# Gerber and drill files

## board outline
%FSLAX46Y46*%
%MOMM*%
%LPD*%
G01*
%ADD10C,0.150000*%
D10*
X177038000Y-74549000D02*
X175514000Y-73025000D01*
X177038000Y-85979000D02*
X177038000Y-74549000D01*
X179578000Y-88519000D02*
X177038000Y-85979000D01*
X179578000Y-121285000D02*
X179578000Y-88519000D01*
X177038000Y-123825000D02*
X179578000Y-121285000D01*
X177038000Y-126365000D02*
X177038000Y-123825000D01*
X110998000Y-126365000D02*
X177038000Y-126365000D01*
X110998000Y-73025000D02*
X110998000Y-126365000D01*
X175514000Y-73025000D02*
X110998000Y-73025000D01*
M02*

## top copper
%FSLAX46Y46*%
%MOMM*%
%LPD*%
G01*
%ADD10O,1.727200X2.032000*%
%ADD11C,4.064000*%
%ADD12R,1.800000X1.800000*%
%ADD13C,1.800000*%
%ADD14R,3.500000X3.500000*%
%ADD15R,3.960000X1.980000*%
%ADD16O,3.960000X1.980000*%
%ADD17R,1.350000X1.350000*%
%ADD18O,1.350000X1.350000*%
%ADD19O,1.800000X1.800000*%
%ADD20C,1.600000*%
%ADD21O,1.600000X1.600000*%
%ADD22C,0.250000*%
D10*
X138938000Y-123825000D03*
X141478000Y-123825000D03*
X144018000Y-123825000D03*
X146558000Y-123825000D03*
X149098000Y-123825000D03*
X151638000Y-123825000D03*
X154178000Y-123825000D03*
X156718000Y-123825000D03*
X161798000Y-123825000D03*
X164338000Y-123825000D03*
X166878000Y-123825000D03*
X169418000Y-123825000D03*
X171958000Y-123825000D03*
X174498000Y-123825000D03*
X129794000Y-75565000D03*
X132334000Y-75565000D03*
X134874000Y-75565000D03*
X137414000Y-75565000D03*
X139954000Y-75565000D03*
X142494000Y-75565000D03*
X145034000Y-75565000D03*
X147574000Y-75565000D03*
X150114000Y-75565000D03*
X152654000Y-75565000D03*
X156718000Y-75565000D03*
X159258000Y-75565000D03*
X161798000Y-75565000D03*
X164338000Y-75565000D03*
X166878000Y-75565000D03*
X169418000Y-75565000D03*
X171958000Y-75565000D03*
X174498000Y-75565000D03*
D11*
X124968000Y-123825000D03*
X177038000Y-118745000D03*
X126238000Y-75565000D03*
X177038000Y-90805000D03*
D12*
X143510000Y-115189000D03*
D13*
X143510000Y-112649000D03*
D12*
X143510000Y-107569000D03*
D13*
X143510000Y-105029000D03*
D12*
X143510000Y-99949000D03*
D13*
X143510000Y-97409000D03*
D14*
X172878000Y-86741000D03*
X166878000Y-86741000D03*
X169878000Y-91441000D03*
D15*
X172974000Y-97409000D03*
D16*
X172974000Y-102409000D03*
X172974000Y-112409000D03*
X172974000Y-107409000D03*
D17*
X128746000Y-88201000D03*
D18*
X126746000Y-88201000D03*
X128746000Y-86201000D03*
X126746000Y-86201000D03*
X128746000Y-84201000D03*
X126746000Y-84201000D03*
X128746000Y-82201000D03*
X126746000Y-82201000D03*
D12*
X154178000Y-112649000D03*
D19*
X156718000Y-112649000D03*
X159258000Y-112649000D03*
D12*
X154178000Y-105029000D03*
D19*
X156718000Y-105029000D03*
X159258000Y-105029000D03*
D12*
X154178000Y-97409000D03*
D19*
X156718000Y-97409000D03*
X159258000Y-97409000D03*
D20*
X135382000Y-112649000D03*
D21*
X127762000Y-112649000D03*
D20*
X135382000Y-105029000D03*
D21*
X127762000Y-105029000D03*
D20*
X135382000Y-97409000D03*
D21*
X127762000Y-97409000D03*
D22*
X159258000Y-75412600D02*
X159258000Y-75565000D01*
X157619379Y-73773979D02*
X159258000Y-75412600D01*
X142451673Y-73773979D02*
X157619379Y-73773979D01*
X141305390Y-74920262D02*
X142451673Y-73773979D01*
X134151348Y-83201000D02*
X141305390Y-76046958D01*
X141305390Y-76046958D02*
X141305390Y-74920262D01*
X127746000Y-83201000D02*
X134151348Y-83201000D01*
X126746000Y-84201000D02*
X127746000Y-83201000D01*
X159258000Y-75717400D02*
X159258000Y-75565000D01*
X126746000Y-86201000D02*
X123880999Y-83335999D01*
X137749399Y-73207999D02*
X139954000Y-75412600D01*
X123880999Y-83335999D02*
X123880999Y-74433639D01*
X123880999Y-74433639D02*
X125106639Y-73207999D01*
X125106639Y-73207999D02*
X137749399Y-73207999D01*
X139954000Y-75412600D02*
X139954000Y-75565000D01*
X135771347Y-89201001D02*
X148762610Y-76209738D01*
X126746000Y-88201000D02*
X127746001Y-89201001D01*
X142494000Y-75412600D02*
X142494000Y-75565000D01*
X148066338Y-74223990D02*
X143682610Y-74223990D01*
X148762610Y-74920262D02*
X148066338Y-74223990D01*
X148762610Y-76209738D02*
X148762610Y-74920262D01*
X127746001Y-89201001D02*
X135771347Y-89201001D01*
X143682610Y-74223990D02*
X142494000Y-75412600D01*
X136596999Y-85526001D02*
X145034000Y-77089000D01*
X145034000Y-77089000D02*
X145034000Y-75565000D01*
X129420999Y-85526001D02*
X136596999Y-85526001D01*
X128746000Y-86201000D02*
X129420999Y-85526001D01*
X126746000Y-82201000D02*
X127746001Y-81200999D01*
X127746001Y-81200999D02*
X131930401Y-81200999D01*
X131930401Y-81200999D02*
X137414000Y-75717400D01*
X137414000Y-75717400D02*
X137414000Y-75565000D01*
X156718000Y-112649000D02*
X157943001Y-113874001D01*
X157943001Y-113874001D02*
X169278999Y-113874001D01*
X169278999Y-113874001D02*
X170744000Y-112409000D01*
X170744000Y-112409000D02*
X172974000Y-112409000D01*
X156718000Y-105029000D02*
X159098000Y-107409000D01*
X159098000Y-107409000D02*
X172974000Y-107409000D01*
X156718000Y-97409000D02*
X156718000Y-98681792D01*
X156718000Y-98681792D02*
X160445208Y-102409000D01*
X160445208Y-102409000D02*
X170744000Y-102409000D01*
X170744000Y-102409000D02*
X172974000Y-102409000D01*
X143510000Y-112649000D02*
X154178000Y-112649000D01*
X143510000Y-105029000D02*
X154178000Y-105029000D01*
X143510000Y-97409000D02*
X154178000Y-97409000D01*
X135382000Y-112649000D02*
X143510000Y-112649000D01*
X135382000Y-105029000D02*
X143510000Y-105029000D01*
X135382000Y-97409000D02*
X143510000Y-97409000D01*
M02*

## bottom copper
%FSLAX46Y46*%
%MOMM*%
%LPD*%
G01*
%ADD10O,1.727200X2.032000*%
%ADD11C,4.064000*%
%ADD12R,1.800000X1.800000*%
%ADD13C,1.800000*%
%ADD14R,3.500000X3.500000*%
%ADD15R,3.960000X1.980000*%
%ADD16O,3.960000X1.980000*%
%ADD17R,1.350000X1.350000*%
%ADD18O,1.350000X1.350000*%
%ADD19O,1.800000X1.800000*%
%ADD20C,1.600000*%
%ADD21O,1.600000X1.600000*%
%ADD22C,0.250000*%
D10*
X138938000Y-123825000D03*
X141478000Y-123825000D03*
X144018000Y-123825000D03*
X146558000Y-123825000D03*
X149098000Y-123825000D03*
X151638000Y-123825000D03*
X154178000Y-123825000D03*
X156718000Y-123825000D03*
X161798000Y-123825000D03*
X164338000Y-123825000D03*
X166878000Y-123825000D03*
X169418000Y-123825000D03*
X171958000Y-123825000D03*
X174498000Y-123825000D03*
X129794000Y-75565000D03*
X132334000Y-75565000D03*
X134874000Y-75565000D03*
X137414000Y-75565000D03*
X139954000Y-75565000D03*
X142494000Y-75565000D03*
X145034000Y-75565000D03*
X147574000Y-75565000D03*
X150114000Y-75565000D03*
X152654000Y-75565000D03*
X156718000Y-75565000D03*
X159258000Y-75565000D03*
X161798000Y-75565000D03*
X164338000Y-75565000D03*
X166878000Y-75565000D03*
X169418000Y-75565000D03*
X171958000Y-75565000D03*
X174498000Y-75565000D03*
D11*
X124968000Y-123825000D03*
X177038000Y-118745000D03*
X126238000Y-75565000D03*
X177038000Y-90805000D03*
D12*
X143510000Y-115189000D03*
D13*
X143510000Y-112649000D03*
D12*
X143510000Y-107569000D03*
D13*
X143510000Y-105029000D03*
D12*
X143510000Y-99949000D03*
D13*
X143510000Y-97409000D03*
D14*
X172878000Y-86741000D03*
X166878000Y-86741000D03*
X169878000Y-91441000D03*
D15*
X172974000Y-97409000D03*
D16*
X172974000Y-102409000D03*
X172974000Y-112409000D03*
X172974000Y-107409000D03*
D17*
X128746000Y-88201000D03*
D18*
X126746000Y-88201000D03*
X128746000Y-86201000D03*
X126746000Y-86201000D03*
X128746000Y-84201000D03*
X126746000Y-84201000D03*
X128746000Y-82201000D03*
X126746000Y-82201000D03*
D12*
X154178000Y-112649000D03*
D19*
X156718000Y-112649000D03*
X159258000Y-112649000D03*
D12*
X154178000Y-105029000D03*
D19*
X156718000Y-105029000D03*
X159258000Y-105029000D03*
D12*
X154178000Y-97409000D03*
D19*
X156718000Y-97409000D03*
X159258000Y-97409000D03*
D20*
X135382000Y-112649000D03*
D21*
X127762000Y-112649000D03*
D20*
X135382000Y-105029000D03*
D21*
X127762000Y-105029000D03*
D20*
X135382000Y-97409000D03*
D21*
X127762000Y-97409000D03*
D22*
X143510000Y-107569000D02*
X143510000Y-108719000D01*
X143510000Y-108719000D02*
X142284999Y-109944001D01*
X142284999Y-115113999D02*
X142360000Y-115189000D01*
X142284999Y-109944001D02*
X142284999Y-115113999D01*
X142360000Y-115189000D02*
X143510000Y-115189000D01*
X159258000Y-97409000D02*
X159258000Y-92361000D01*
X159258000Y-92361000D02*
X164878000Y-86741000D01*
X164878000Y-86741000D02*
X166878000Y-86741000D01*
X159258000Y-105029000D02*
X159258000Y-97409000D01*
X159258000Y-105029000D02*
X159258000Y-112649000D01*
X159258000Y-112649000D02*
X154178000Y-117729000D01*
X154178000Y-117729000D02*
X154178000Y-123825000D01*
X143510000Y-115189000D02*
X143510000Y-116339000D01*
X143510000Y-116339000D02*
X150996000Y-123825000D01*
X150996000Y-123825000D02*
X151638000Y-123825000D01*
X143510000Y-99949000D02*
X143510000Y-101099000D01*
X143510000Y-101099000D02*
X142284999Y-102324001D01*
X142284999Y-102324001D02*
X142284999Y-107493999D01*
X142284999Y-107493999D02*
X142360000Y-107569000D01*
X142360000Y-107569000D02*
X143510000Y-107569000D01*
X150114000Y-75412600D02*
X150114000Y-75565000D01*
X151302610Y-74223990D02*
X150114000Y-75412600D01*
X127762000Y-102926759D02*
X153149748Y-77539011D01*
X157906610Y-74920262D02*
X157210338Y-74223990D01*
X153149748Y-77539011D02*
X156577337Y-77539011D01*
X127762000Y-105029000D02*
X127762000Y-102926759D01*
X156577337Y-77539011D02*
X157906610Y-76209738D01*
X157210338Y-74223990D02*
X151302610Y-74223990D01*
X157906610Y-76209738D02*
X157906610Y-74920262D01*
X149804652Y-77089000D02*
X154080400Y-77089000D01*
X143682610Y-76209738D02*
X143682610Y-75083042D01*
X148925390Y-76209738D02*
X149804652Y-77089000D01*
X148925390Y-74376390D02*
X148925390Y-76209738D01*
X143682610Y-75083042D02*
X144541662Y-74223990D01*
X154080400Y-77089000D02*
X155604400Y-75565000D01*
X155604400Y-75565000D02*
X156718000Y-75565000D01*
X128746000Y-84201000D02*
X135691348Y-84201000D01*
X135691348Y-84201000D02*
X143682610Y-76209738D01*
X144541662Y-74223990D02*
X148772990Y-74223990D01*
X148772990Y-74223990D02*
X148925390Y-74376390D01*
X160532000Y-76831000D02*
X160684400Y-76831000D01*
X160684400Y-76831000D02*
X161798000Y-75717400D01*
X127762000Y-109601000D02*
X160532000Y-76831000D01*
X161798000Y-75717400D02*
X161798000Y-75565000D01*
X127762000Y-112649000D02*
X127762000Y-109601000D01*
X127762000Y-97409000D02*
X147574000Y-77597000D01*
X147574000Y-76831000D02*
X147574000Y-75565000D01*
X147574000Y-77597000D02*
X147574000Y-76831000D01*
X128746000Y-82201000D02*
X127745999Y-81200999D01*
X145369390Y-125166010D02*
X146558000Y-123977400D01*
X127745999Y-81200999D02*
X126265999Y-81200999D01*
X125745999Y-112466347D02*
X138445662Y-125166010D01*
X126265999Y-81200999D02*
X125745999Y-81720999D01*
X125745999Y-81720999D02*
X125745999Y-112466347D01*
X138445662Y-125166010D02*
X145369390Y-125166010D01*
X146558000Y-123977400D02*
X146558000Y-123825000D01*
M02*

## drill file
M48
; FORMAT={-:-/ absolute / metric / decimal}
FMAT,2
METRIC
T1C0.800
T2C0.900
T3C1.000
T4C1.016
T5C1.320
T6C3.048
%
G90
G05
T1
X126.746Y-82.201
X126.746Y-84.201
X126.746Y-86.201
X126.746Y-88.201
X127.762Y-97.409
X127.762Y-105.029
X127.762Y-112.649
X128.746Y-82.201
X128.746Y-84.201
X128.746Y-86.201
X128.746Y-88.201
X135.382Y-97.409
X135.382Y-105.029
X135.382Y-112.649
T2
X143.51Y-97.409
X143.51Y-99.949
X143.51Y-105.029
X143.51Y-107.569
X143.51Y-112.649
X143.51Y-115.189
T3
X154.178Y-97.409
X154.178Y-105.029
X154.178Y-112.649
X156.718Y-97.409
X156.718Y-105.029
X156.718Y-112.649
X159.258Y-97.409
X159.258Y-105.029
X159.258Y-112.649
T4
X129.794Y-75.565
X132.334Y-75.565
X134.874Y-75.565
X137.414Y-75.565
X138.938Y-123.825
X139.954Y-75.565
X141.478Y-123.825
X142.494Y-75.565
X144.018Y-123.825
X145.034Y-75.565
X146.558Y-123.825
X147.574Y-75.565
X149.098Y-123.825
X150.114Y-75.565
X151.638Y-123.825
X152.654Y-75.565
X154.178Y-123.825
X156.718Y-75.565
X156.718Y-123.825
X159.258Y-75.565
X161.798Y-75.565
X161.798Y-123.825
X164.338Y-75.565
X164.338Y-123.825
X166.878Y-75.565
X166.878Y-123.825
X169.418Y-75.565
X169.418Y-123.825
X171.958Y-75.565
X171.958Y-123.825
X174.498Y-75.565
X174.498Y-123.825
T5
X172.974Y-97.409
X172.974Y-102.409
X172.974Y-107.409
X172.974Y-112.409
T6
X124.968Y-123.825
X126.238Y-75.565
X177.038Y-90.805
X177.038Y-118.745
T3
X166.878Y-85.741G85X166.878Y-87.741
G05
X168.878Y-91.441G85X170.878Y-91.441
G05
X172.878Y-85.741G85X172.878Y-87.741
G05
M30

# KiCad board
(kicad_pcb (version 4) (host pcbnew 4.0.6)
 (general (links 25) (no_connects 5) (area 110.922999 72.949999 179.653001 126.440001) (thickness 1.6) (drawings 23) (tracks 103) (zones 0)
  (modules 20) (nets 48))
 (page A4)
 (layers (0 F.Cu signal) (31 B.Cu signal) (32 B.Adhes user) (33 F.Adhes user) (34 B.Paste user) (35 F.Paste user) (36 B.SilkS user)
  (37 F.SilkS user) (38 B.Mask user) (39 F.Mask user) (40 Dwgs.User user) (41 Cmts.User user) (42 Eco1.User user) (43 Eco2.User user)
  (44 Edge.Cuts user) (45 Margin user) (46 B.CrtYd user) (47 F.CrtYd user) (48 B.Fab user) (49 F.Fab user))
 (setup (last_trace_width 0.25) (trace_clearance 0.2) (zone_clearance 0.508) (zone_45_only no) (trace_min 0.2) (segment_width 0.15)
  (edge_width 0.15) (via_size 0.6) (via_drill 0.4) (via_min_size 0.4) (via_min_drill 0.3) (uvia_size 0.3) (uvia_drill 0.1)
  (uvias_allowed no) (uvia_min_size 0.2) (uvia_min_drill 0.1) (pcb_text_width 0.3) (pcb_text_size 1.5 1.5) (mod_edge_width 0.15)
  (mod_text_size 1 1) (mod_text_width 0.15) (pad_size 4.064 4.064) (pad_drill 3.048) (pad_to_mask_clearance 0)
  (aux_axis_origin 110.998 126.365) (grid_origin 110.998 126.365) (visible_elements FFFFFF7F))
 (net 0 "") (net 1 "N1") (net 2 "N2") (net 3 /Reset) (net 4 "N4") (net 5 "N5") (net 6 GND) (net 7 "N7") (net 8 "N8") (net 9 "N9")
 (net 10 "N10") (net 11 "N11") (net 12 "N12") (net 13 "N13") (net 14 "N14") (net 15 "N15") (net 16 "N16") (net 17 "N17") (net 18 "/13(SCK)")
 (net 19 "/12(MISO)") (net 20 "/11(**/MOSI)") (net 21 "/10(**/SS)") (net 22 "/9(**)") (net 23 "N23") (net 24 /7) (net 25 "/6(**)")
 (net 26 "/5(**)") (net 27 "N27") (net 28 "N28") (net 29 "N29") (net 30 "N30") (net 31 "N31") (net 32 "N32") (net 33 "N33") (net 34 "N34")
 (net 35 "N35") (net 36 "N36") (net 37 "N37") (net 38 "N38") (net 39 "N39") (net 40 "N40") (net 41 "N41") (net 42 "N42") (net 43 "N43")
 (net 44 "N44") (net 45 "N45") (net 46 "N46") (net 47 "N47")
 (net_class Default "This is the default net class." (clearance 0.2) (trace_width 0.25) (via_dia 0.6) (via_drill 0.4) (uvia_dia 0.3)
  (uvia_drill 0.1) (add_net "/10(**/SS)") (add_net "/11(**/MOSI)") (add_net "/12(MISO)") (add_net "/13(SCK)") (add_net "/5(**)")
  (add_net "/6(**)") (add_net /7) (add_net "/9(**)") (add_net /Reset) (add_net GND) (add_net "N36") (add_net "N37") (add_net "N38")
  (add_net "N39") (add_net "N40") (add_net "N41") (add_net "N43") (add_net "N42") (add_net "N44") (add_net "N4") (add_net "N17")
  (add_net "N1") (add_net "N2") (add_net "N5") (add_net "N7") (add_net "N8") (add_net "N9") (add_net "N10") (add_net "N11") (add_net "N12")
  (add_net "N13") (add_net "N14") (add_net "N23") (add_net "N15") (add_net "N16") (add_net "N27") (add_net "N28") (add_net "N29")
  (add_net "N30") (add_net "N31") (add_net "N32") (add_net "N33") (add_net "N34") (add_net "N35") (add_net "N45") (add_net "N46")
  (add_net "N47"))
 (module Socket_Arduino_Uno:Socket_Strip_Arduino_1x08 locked (layer F.Cu) (at 138.938 123.825)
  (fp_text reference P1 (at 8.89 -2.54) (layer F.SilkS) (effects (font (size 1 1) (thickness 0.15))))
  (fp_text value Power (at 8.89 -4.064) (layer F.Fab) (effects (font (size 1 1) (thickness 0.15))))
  (pad 1 thru_hole oval (at 0 0) (size 1.7272 2.032) (drill 1.016) (layers *.Cu *.Mask F.SilkS) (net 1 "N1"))
  (pad 2 thru_hole oval (at 2.54 0) (size 1.7272 2.032) (drill 1.016) (layers *.Cu *.Mask F.SilkS) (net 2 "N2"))
  (pad 3 thru_hole oval (at 5.08 0) (size 1.7272 2.032) (drill 1.016) (layers *.Cu *.Mask F.SilkS) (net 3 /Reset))
  (pad 4 thru_hole oval (at 7.62 0) (size 1.7272 2.032) (drill 1.016) (layers *.Cu *.Mask F.SilkS) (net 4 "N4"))
  (pad 5 thru_hole oval (at 10.16 0) (size 1.7272 2.032) (drill 1.016) (layers *.Cu *.Mask F.SilkS) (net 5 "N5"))
  (pad 6 thru_hole oval (at 12.7 0) (size 1.7272 2.032) (drill 1.016) (layers *.Cu *.Mask F.SilkS) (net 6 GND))
  (pad 7 thru_hole oval (at 15.24 0) (size 1.7272 2.032) (drill 1.016) (layers *.Cu *.Mask F.SilkS) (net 6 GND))
  (pad 8 thru_hole oval (at 17.78 0) (size 1.7272 2.032) (drill 1.016) (layers *.Cu *.Mask F.SilkS) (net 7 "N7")))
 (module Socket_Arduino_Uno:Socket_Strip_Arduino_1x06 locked (layer F.Cu) (at 161.798 123.825)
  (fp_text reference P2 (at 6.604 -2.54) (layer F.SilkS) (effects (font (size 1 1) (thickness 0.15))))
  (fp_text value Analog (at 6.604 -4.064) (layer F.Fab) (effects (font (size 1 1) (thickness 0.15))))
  (pad 1 thru_hole oval (at 0 0) (size 1.7272 2.032) (drill 1.016) (layers *.Cu *.Mask F.SilkS) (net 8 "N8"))
  (pad 2 thru_hole oval (at 2.54 0) (size 1.7272 2.032) (drill 1.016) (layers *.Cu *.Mask F.SilkS) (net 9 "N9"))
  (pad 3 thru_hole oval (at 5.08 0) (size 1.7272 2.032) (drill 1.016) (layers *.Cu *.Mask F.SilkS) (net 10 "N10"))
  (pad 4 thru_hole oval (at 7.62 0) (size 1.7272 2.032) (drill 1.016) (layers *.Cu *.Mask F.SilkS) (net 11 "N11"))
  (pad 5 thru_hole oval (at 10.16 0) (size 1.7272 2.032) (drill 1.016) (layers *.Cu *.Mask F.SilkS) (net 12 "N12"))
  (pad 6 thru_hole oval (at 12.7 0) (size 1.7272 2.032) (drill 1.016) (layers *.Cu *.Mask F.SilkS) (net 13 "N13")))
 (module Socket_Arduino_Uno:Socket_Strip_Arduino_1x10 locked (layer F.Cu) (at 129.794 75.565)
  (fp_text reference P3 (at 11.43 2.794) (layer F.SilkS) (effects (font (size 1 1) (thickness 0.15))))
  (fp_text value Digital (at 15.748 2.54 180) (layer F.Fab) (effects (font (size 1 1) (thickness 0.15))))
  (pad 1 thru_hole oval (at 0 0) (size 1.7272 2.032) (drill 1.016) (layers *.Cu *.Mask F.SilkS) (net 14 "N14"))
  (pad 2 thru_hole oval (at 2.54 0) (size 1.7272 2.032) (drill 1.016) (layers *.Cu *.Mask F.SilkS) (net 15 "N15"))
  (pad 3 thru_hole oval (at 5.08 0) (size 1.7272 2.032) (drill 1.016) (layers *.Cu *.Mask F.SilkS) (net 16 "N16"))
  (pad 4 thru_hole oval (at 7.62 0) (size 1.7272 2.032) (drill 1.016) (layers *.Cu *.Mask F.SilkS) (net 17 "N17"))
  (pad 5 thru_hole oval (at 10.16 0) (size 1.7272 2.032) (drill 1.016) (layers *.Cu *.Mask F.SilkS) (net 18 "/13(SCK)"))
  (pad 6 thru_hole oval (at 12.7 0) (size 1.7272 2.032) (drill 1.016) (layers *.Cu *.Mask F.SilkS) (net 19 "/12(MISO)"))
  (pad 7 thru_hole oval (at 15.24 0) (size 1.7272 2.032) (drill 1.016) (layers *.Cu *.Mask F.SilkS) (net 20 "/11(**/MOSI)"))
  (pad 8 thru_hole oval (at 17.78 0) (size 1.7272 2.032) (drill 1.016) (layers *.Cu *.Mask F.SilkS) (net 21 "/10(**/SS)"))
  (pad 9 thru_hole oval (at 20.32 0) (size 1.7272 2.032) (drill 1.016) (layers *.Cu *.Mask F.SilkS) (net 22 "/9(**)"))
  (pad 10 thru_hole oval (at 22.86 0) (size 1.7272 2.032) (drill 1.016) (layers *.Cu *.Mask F.SilkS) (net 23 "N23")))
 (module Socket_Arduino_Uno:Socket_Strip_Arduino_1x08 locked (layer F.Cu) (at 156.718 75.565)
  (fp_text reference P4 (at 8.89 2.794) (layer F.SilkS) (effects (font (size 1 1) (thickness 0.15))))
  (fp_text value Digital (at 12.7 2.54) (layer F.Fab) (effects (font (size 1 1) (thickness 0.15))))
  (pad 1 thru_hole oval (at 0 0) (size 1.7272 2.032) (drill 1.016) (layers *.Cu *.Mask F.SilkS) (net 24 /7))
  (pad 2 thru_hole oval (at 2.54 0) (size 1.7272 2.032) (drill 1.016) (layers *.Cu *.Mask F.SilkS) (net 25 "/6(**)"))
  (pad 3 thru_hole oval (at 5.08 0) (size 1.7272 2.032) (drill 1.016) (layers *.Cu *.Mask F.SilkS) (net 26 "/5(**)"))
  (pad 4 thru_hole oval (at 7.62 0) (size 1.7272 2.032) (drill 1.016) (layers *.Cu *.Mask F.SilkS) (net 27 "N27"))
  (pad 5 thru_hole oval (at 10.16 0) (size 1.7272 2.032) (drill 1.016) (layers *.Cu *.Mask F.SilkS) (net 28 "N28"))
  (pad 6 thru_hole oval (at 12.7 0) (size 1.7272 2.032) (drill 1.016) (layers *.Cu *.Mask F.SilkS) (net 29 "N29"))
  (pad 7 thru_hole oval (at 15.24 0) (size 1.7272 2.032) (drill 1.016) (layers *.Cu *.Mask F.SilkS) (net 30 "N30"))
  (pad 8 thru_hole oval (at 17.78 0) (size 1.7272 2.032) (drill 1.016) (layers *.Cu *.Mask F.SilkS) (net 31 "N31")))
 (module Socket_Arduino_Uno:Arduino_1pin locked (layer F.Cu) (at 124.968 123.825)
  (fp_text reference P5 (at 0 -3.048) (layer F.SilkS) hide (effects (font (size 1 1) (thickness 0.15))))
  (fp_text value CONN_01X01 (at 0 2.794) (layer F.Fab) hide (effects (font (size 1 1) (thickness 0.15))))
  (pad 1 thru_hole circle (at 0 0) (size 4.064 4.064) (drill 3.048) (layers *.Cu *.Mask F.SilkS) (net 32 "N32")))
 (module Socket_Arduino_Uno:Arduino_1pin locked (layer F.Cu) (at 177.038 118.745)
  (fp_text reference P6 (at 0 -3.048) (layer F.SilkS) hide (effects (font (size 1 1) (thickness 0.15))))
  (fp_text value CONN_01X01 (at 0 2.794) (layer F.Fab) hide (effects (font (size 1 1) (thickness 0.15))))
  (pad 1 thru_hole circle (at 0 0) (size 4.064 4.064) (drill 3.048) (layers *.Cu *.Mask F.SilkS) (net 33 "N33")))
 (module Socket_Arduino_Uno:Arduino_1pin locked (layer F.Cu) (at 126.238 75.565)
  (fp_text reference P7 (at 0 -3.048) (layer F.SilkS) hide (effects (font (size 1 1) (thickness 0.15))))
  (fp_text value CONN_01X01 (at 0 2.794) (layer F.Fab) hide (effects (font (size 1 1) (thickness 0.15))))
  (pad 1 thru_hole circle (at 0 0) (size 4.064 4.064) (drill 3.048) (layers *.Cu *.Mask F.SilkS) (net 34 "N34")))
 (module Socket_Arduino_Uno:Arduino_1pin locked (layer F.Cu) (at 177.038 90.805)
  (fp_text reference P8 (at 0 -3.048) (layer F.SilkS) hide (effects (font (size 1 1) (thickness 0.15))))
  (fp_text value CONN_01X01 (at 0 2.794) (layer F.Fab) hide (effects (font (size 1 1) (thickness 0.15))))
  (pad 1 thru_hole circle (at 0 0) (size 4.064 4.064) (drill 3.048) (layers *.Cu *.Mask F.SilkS) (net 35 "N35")))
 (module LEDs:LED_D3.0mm (layer F.Cu) (at 143.51 115.189 90)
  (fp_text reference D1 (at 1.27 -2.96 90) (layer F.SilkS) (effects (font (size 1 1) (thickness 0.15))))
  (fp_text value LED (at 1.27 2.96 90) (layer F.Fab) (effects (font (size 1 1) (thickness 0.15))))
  (pad 1 thru_hole rect (at 0 0 90) (size 1.8 1.8) (drill 0.9) (layers *.Cu *.Mask) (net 6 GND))
  (pad 2 thru_hole circle (at 2.54 0 90) (size 1.8 1.8) (drill 0.9) (layers *.Cu *.Mask) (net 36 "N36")))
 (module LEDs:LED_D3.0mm (layer F.Cu) (at 143.51 107.569 90)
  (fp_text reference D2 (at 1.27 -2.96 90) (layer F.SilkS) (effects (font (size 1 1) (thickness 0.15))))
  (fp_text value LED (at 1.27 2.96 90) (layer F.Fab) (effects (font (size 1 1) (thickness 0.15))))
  (pad 1 thru_hole rect (at 0 0 90) (size 1.8 1.8) (drill 0.9) (layers *.Cu *.Mask) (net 6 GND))
  (pad 2 thru_hole circle (at 2.54 0 90) (size 1.8 1.8) (drill 0.9) (layers *.Cu *.Mask) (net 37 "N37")))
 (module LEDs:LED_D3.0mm (layer F.Cu) (at 143.51 99.949 90)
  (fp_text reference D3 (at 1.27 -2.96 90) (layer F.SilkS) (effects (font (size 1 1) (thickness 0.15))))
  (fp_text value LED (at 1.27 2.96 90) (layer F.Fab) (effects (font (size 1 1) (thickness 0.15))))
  (pad 1 thru_hole rect (at 0 0 90) (size 1.8 1.8) (drill 0.9) (layers *.Cu *.Mask) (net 6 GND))
  (pad 2 thru_hole circle (at 2.54 0 90) (size 1.8 1.8) (drill 0.9) (layers *.Cu *.Mask) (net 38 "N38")))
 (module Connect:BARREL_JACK (layer F.Cu) (at 172.878 86.741)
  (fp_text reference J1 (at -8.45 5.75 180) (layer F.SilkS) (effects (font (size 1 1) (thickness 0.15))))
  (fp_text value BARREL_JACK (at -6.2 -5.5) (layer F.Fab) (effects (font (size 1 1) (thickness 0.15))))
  (pad 1 thru_hole rect (at 0 0) (size 3.5 3.5) (drill oval 1 3) (layers *.Cu *.Mask) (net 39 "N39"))
  (pad 2 thru_hole rect (at -6 0) (size 3.5 3.5) (drill oval 1 3) (layers *.Cu *.Mask) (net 6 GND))
  (pad 3 thru_hole rect (at -3 4.7) (size 3.5 3.5) (drill oval 3 1) (layers *.Cu *.Mask) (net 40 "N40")))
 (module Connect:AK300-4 (layer F.Cu) (at 172.974 97.409 270)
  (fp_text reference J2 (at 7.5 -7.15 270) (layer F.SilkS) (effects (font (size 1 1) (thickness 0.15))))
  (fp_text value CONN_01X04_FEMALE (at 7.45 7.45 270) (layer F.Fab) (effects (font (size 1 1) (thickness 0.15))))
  (pad 1 thru_hole rect (at 0 0 270) (size 1.98 3.96) (drill 1.32) (layers *.Cu F.Paste F.Mask) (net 39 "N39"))
  (pad 2 thru_hole oval (at 5 0 270) (size 1.98 3.96) (drill 1.32) (layers *.Cu F.Paste F.Mask) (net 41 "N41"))
  (pad 4 thru_hole oval (at 15 0 270) (size 1.98 3.96) (drill 1.32) (layers *.Cu F.Paste F.Mask) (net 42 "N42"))
  (pad 3 thru_hole oval (at 10 0 270) (size 1.98 3.96) (drill 1.32) (layers *.Cu *.Mask) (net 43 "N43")))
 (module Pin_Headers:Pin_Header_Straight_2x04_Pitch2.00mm (layer F.Cu) (at 128.746 88.201 180)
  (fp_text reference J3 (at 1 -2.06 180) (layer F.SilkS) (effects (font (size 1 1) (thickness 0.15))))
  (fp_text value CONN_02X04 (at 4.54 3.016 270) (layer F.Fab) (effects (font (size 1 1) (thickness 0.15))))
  (pad 1 thru_hole rect (at 0 0 180) (size 1.35 1.35) (drill 0.8) (layers *.Cu *.Mask) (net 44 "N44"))
  (pad 2 thru_hole oval (at 2 0 180) (size 1.35 1.35) (drill 0.8) (layers *.Cu *.Mask) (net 19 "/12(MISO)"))
  (pad 3 thru_hole oval (at 0 2 180) (size 1.35 1.35) (drill 0.8) (layers *.Cu *.Mask) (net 20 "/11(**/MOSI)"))
  (pad 4 thru_hole oval (at 2 2 180) (size 1.35 1.35) (drill 0.8) (layers *.Cu *.Mask) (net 18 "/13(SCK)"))
  (pad 5 thru_hole oval (at 0 4 180) (size 1.35 1.35) (drill 0.8) (layers *.Cu *.Mask) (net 24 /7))
  (pad 6 thru_hole oval (at 2 4 180) (size 1.35 1.35) (drill 0.8) (layers *.Cu *.Mask) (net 25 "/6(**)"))
  (pad 7 thru_hole oval (at 0 6 180) (size 1.35 1.35) (drill 0.8) (layers *.Cu *.Mask) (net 4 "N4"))
  (pad 8 thru_hole oval (at 2 6 180) (size 1.35 1.35) (drill 0.8) (layers *.Cu *.Mask) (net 17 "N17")))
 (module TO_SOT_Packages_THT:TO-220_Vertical (layer F.Cu) (at 154.178 112.649)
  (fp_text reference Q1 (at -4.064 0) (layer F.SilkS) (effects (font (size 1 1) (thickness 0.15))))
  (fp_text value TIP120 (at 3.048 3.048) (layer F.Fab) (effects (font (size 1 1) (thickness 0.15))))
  (pad 1 thru_hole rect (at 0 0) (size 1.8 1.8) (drill 1) (layers *.Cu *.Mask) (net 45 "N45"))
  (pad 2 thru_hole oval (at 2.54 0) (size 1.8 1.8) (drill 1) (layers *.Cu *.Mask) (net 42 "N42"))
  (pad 3 thru_hole oval (at 5.08 0) (size 1.8 1.8) (drill 1) (layers *.Cu *.Mask) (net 6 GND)))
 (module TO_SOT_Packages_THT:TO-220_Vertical (layer F.Cu) (at 154.178 105.029)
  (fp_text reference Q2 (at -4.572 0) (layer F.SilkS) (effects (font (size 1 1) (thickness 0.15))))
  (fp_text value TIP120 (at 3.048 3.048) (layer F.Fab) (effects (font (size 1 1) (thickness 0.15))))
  (pad 1 thru_hole rect (at 0 0) (size 1.8 1.8) (drill 1) (layers *.Cu *.Mask) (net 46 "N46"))
  (pad 2 thru_hole oval (at 2.54 0) (size 1.8 1.8) (drill 1) (layers *.Cu *.Mask) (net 43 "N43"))
  (pad 3 thru_hole oval (at 5.08 0) (size 1.8 1.8) (drill 1) (layers *.Cu *.Mask) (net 6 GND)))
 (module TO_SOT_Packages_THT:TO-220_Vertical (layer F.Cu) (at 154.178 97.409)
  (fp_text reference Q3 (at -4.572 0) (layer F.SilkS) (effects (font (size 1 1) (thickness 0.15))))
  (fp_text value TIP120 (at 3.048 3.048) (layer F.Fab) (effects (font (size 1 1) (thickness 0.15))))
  (pad 1 thru_hole rect (at 0 0) (size 1.8 1.8) (drill 1) (layers *.Cu *.Mask) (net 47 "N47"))
  (pad 2 thru_hole oval (at 2.54 0) (size 1.8 1.8) (drill 1) (layers *.Cu *.Mask) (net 41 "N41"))
  (pad 3 thru_hole oval (at 5.08 0) (size 1.8 1.8) (drill 1) (layers *.Cu *.Mask) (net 6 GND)))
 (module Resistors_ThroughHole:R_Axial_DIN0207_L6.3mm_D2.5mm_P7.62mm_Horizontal (layer F.Cu) (at 135.382 112.649 180)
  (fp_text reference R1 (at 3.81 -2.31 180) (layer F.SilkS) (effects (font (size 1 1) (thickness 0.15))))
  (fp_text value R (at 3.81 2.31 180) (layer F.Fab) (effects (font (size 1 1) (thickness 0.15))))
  (pad 1 thru_hole circle (at 0 0 180) (size 1.6 1.6) (drill 0.8) (layers *.Cu *.Mask) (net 45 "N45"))
  (pad 2 thru_hole oval (at 7.62 0 180) (size 1.6 1.6) (drill 0.8) (layers *.Cu *.Mask) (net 26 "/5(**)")))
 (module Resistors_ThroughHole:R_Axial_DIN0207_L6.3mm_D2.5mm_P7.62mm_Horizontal (layer F.Cu) (at 135.382 105.029 180)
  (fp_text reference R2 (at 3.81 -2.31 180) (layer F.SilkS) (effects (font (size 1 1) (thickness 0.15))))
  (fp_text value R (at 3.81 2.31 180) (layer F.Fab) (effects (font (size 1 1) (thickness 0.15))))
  (pad 1 thru_hole circle (at 0 0 180) (size 1.6 1.6) (drill 0.8) (layers *.Cu *.Mask) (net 46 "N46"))
  (pad 2 thru_hole oval (at 7.62 0 180) (size 1.6 1.6) (drill 0.8) (layers *.Cu *.Mask) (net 22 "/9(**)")))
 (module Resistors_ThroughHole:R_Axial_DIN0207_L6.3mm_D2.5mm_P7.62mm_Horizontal (layer F.Cu) (at 135.382 97.409 180)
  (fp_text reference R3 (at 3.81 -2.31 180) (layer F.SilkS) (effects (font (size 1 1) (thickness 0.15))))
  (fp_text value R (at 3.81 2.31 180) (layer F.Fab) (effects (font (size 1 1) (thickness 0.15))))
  (pad 1 thru_hole circle (at 0 0 180) (size 1.6 1.6) (drill 0.8) (layers *.Cu *.Mask) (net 47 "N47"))
  (pad 2 thru_hole oval (at 7.62 0 180) (size 1.6 1.6) (drill 0.8) (layers *.Cu *.Mask) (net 21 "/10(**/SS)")))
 (gr_line (start 177.038 74.549) (end 175.514 73.025) (angle 90) (layer Edge.Cuts) (width 0.15))
 (gr_line (start 177.038 85.979) (end 177.038 74.549) (angle 90) (layer Edge.Cuts) (width 0.15))
 (gr_line (start 179.578 88.519) (end 177.038 85.979) (angle 90) (layer Edge.Cuts) (width 0.15))
 (gr_line (start 179.578 121.285) (end 179.578 88.519) (angle 90) (layer Edge.Cuts) (width 0.15))
 (gr_line (start 177.038 123.825) (end 179.578 121.285) (angle 90) (layer Edge.Cuts) (width 0.15))
 (gr_line (start 177.038 126.365) (end 177.038 123.825) (angle 90) (layer Edge.Cuts) (width 0.15))
 (gr_line (start 110.998 126.365) (end 177.038 126.365) (angle 90) (layer Edge.Cuts) (width 0.15))
 (gr_line (start 110.998 73.025) (end 110.998 126.365) (angle 90) (layer Edge.Cuts) (width 0.15))
 (gr_line (start 175.514 73.025) (end 110.998 73.025) (angle 90) (layer Edge.Cuts) (width 0.15))
 (segment (start 143.51 107.569) (end 143.51 108.719) (width 0.25) (layer B.Cu) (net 6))
 (segment (start 143.51 108.719) (end 142.284999 109.944001) (width 0.25) (layer B.Cu) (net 6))
 (segment (start 142.284999 115.113999) (end 142.36 115.189) (width 0.25) (layer B.Cu) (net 6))
 (segment (start 142.284999 109.944001) (end 142.284999 115.113999) (width 0.25) (layer B.Cu) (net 6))
 (segment (start 142.36 115.189) (end 143.51 115.189) (width 0.25) (layer B.Cu) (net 6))
 (segment (start 159.258 97.409) (end 159.258 92.361) (width 0.25) (layer B.Cu) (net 6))
 (segment (start 159.258 92.361) (end 164.878 86.741) (width 0.25) (layer B.Cu) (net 6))
 (segment (start 164.878 86.741) (end 166.878 86.741) (width 0.25) (layer B.Cu) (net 6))
 (segment (start 159.258 105.029) (end 159.258 97.409) (width 0.25) (layer B.Cu) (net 6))
 (segment (start 159.258 105.029) (end 159.258 112.649) (width 0.25) (layer B.Cu) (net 6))
 (segment (start 159.258 112.649) (end 154.178 117.729) (width 0.25) (layer B.Cu) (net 6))
 (segment (start 154.178 117.729) (end 154.178 123.825) (width 0.25) (layer B.Cu) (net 6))
 (segment (start 143.51 115.189) (end 143.51 116.339) (width 0.25) (layer B.Cu) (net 6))
 (segment (start 143.51 116.339) (end 150.996 123.825) (width 0.25) (layer B.Cu) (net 6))
 (segment (start 150.996 123.825) (end 151.638 123.825) (width 0.25) (layer B.Cu) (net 6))
 (segment (start 143.51 99.949) (end 143.51 101.099) (width 0.25) (layer B.Cu) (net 6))
 (segment (start 143.51 101.099) (end 142.284999 102.324001) (width 0.25) (layer B.Cu) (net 6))
 (segment (start 142.284999 102.324001) (end 142.284999 107.493999) (width 0.25) (layer B.Cu) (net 6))
 (segment (start 142.284999 107.493999) (end 142.36 107.569) (width 0.25) (layer B.Cu) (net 6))
 (segment (start 142.36 107.569) (end 143.51 107.569) (width 0.25) (layer B.Cu) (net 6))
 (segment (start 150.114 75.4126) (end 150.114 75.565) (width 0.25) (layer B.Cu) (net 22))
 (segment (start 151.30261 74.22399) (end 150.114 75.4126) (width 0.25) (layer B.Cu) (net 22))
 (segment (start 127.762 102.926759) (end 153.149748 77.539011) (width 0.25) (layer B.Cu) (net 22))
 (segment (start 157.90661 74.920262) (end 157.210338 74.22399) (width 0.25) (layer B.Cu) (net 22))
 (segment (start 153.149748 77.539011) (end 156.577337 77.539011) (width 0.25) (layer B.Cu) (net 22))
 (segment (start 127.762 105.029) (end 127.762 102.926759) (width 0.25) (layer B.Cu) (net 22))
 (segment (start 156.577337 77.539011) (end 157.90661 76.209738) (width 0.25) (layer B.Cu) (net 22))
 (segment (start 157.210338 74.22399) (end 151.30261 74.22399) (width 0.25) (layer B.Cu) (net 22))
 (segment (start 157.90661 76.209738) (end 157.90661 74.920262) (width 0.25) (layer B.Cu) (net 22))
 (segment (start 149.804652 77.089) (end 154.0804 77.089) (width 0.25) (layer B.Cu) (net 24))
 (segment (start 143.68261 76.209738) (end 143.68261 75.083042) (width 0.25) (layer B.Cu) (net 24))
 (segment (start 148.92539 76.209738) (end 149.804652 77.089) (width 0.25) (layer B.Cu) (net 24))
 (segment (start 148.92539 74.37639) (end 148.92539 76.209738) (width 0.25) (layer B.Cu) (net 24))
 (segment (start 143.68261 75.083042) (end 144.541662 74.22399) (width 0.25) (layer B.Cu) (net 24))
 (segment (start 154.0804 77.089) (end 155.6044 75.565) (width 0.25) (layer B.Cu) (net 24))
 (segment (start 155.6044 75.565) (end 156.718 75.565) (width 0.25) (layer B.Cu) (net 24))
 (segment (start 128.746 84.201) (end 135.691348 84.201) (width 0.25) (layer B.Cu) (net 24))
 (segment (start 135.691348 84.201) (end 143.68261 76.209738) (width 0.25) (layer B.Cu) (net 24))
 (segment (start 144.541662 74.22399) (end 148.77299 74.22399) (width 0.25) (layer B.Cu) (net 24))
 (segment (start 148.77299 74.22399) (end 148.92539 74.37639) (width 0.25) (layer B.Cu) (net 24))
 (segment (start 159.258 75.4126) (end 159.258 75.565) (width 0.25) (layer F.Cu) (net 25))
 (segment (start 157.619379 73.773979) (end 159.258 75.4126) (width 0.25) (layer F.Cu) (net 25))
 (segment (start 142.451673 73.773979) (end 157.619379 73.773979) (width 0.25) (layer F.Cu) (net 25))
 (segment (start 141.30539 74.920262) (end 142.451673 73.773979) (width 0.25) (layer F.Cu) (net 25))
 (segment (start 134.151348 83.201) (end 141.30539 76.046958) (width 0.25) (layer F.Cu) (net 25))
 (segment (start 141.30539 76.046958) (end 141.30539 74.920262) (width 0.25) (layer F.Cu) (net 25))
 (segment (start 127.746 83.201) (end 134.151348 83.201) (width 0.25) (layer F.Cu) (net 25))
 (segment (start 126.746 84.201) (end 127.746 83.201) (width 0.25) (layer F.Cu) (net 25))
 (segment (start 159.258 75.7174) (end 159.258 75.565) (width 0.25) (layer F.Cu) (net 25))
 (segment (start 160.532 76.831) (end 160.6844 76.831) (width 0.25) (layer B.Cu) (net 26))
 (segment (start 160.6844 76.831) (end 161.798 75.7174) (width 0.25) (layer B.Cu) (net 26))
 (segment (start 127.762 109.601) (end 160.532 76.831) (width 0.25) (layer B.Cu) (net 26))
 (segment (start 161.798 75.7174) (end 161.798 75.565) (width 0.25) (layer B.Cu) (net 26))
 (segment (start 127.762 112.649) (end 127.762 109.601) (width 0.25) (layer B.Cu) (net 26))
 (segment (start 126.746 86.201) (end 123.880999 83.335999) (width 0.25) (layer F.Cu) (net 18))
 (segment (start 137.749399 73.207999) (end 139.954 75.4126) (width 0.25) (layer F.Cu) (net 18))
 (segment (start 123.880999 83.335999) (end 123.880999 74.433639) (width 0.25) (layer F.Cu) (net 18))
 (segment (start 123.880999 74.433639) (end 125.106639 73.207999) (width 0.25) (layer F.Cu) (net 18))
 (segment (start 125.106639 73.207999) (end 137.749399 73.207999) (width 0.25) (layer F.Cu) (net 18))
 (segment (start 139.954 75.4126) (end 139.954 75.565) (width 0.25) (layer F.Cu) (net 18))
 (segment (start 127.762 97.409) (end 147.574 77.597) (width 0.25) (layer B.Cu) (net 21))
 (segment (start 147.574 76.831) (end 147.574 75.565) (width 0.25) (layer B.Cu) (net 21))
 (segment (start 147.574 77.597) (end 147.574 76.831) (width 0.25) (layer B.Cu) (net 21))
 (segment (start 135.771347 89.201001) (end 148.76261 76.209738) (width 0.25) (layer F.Cu) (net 19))
 (segment (start 126.746 88.201) (end 127.746001 89.201001) (width 0.25) (layer F.Cu) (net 19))
 (segment (start 142.494 75.4126) (end 142.494 75.565) (width 0.25) (layer F.Cu) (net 19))
 (segment (start 148.066338 74.22399) (end 143.68261 74.22399) (width 0.25) (layer F.Cu) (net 19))
 (segment (start 148.76261 74.920262) (end 148.066338 74.22399) (width 0.25) (layer F.Cu) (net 19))
 (segment (start 148.76261 76.209738) (end 148.76261 74.920262) (width 0.25) (layer F.Cu) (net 19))
 (segment (start 127.746001 89.201001) (end 135.771347 89.201001) (width 0.25) (layer F.Cu) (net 19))
 (segment (start 143.68261 74.22399) (end 142.494 75.4126) (width 0.25) (layer F.Cu) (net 19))
 (segment (start 136.596999 85.526001) (end 145.034 77.089) (width 0.25) (layer F.Cu) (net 20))
 (segment (start 145.034 77.089) (end 145.034 75.565) (width 0.25) (layer F.Cu) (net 20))
 (segment (start 129.420999 85.526001) (end 136.596999 85.526001) (width 0.25) (layer F.Cu) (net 20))
 (segment (start 128.746 86.201) (end 129.420999 85.526001) (width 0.25) (layer F.Cu) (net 20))
 (segment (start 128.746 82.201) (end 127.745999 81.200999) (width 0.25) (layer B.Cu) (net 4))
 (segment (start 145.36939 125.16601) (end 146.558 123.9774) (width 0.25) (layer B.Cu) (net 4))
 (segment (start 127.745999 81.200999) (end 126.265999 81.200999) (width 0.25) (layer B.Cu) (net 4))
 (segment (start 125.745999 112.466347) (end 138.445662 125.16601) (width 0.25) (layer B.Cu) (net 4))
 (segment (start 126.265999 81.200999) (end 125.745999 81.720999) (width 0.25) (layer B.Cu) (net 4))
 (segment (start 125.745999 81.720999) (end 125.745999 112.466347) (width 0.25) (layer B.Cu) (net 4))
 (segment (start 138.445662 125.16601) (end 145.36939 125.16601) (width 0.25) (layer B.Cu) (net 4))
 (segment (start 146.558 123.9774) (end 146.558 123.825) (width 0.25) (layer B.Cu) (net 4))
 (segment (start 126.746 82.201) (end 127.746001 81.200999) (width 0.25) (layer F.Cu) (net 17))
 (segment (start 127.746001 81.200999) (end 131.930401 81.200999) (width 0.25) (layer F.Cu) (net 17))
 (segment (start 131.930401 81.200999) (end 137.414 75.7174) (width 0.25) (layer F.Cu) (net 17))
 (segment (start 137.414 75.7174) (end 137.414 75.565) (width 0.25) (layer F.Cu) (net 17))
 (segment (start 156.718 112.649) (end 157.943001 113.874001) (width 0.25) (layer F.Cu) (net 42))
 (segment (start 157.943001 113.874001) (end 169.278999 113.874001) (width 0.25) (layer F.Cu) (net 42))
 (segment (start 169.278999 113.874001) (end 170.744 112.409) (width 0.25) (layer F.Cu) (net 42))
 (segment (start 170.744 112.409) (end 172.974 112.409) (width 0.25) (layer F.Cu) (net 42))
 (segment (start 156.718 105.029) (end 159.098 107.409) (width 0.25) (layer F.Cu) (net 43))
 (segment (start 159.098 107.409) (end 172.974 107.409) (width 0.25) (layer F.Cu) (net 43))
 (segment (start 156.718 97.409) (end 156.718 98.681792) (width 0.25) (layer F.Cu) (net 41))
 (segment (start 156.718 98.681792) (end 160.445208 102.409) (width 0.25) (layer F.Cu) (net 41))
 (segment (start 160.445208 102.409) (end 170.744 102.409) (width 0.25) (layer F.Cu) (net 41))
 (segment (start 170.744 102.409) (end 172.974 102.409) (width 0.25) (layer F.Cu) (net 41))
 (segment (start 143.51 112.649) (end 154.178 112.649) (width 0.25) (layer F.Cu) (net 36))
 (segment (start 143.51 105.029) (end 154.178 105.029) (width 0.25) (layer F.Cu) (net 37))
 (segment (start 143.51 97.409) (end 154.178 97.409) (width 0.25) (layer F.Cu) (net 38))
 (segment (start 135.382 112.649) (end 143.51 112.649) (width 0.25) (layer F.Cu) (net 45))
 (segment (start 135.382 105.029) (end 143.51 105.029) (width 0.25) (layer F.Cu) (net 46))
 (segment (start 135.382 97.409) (end 143.51 97.409) (width 0.25) (layer F.Cu) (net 47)))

